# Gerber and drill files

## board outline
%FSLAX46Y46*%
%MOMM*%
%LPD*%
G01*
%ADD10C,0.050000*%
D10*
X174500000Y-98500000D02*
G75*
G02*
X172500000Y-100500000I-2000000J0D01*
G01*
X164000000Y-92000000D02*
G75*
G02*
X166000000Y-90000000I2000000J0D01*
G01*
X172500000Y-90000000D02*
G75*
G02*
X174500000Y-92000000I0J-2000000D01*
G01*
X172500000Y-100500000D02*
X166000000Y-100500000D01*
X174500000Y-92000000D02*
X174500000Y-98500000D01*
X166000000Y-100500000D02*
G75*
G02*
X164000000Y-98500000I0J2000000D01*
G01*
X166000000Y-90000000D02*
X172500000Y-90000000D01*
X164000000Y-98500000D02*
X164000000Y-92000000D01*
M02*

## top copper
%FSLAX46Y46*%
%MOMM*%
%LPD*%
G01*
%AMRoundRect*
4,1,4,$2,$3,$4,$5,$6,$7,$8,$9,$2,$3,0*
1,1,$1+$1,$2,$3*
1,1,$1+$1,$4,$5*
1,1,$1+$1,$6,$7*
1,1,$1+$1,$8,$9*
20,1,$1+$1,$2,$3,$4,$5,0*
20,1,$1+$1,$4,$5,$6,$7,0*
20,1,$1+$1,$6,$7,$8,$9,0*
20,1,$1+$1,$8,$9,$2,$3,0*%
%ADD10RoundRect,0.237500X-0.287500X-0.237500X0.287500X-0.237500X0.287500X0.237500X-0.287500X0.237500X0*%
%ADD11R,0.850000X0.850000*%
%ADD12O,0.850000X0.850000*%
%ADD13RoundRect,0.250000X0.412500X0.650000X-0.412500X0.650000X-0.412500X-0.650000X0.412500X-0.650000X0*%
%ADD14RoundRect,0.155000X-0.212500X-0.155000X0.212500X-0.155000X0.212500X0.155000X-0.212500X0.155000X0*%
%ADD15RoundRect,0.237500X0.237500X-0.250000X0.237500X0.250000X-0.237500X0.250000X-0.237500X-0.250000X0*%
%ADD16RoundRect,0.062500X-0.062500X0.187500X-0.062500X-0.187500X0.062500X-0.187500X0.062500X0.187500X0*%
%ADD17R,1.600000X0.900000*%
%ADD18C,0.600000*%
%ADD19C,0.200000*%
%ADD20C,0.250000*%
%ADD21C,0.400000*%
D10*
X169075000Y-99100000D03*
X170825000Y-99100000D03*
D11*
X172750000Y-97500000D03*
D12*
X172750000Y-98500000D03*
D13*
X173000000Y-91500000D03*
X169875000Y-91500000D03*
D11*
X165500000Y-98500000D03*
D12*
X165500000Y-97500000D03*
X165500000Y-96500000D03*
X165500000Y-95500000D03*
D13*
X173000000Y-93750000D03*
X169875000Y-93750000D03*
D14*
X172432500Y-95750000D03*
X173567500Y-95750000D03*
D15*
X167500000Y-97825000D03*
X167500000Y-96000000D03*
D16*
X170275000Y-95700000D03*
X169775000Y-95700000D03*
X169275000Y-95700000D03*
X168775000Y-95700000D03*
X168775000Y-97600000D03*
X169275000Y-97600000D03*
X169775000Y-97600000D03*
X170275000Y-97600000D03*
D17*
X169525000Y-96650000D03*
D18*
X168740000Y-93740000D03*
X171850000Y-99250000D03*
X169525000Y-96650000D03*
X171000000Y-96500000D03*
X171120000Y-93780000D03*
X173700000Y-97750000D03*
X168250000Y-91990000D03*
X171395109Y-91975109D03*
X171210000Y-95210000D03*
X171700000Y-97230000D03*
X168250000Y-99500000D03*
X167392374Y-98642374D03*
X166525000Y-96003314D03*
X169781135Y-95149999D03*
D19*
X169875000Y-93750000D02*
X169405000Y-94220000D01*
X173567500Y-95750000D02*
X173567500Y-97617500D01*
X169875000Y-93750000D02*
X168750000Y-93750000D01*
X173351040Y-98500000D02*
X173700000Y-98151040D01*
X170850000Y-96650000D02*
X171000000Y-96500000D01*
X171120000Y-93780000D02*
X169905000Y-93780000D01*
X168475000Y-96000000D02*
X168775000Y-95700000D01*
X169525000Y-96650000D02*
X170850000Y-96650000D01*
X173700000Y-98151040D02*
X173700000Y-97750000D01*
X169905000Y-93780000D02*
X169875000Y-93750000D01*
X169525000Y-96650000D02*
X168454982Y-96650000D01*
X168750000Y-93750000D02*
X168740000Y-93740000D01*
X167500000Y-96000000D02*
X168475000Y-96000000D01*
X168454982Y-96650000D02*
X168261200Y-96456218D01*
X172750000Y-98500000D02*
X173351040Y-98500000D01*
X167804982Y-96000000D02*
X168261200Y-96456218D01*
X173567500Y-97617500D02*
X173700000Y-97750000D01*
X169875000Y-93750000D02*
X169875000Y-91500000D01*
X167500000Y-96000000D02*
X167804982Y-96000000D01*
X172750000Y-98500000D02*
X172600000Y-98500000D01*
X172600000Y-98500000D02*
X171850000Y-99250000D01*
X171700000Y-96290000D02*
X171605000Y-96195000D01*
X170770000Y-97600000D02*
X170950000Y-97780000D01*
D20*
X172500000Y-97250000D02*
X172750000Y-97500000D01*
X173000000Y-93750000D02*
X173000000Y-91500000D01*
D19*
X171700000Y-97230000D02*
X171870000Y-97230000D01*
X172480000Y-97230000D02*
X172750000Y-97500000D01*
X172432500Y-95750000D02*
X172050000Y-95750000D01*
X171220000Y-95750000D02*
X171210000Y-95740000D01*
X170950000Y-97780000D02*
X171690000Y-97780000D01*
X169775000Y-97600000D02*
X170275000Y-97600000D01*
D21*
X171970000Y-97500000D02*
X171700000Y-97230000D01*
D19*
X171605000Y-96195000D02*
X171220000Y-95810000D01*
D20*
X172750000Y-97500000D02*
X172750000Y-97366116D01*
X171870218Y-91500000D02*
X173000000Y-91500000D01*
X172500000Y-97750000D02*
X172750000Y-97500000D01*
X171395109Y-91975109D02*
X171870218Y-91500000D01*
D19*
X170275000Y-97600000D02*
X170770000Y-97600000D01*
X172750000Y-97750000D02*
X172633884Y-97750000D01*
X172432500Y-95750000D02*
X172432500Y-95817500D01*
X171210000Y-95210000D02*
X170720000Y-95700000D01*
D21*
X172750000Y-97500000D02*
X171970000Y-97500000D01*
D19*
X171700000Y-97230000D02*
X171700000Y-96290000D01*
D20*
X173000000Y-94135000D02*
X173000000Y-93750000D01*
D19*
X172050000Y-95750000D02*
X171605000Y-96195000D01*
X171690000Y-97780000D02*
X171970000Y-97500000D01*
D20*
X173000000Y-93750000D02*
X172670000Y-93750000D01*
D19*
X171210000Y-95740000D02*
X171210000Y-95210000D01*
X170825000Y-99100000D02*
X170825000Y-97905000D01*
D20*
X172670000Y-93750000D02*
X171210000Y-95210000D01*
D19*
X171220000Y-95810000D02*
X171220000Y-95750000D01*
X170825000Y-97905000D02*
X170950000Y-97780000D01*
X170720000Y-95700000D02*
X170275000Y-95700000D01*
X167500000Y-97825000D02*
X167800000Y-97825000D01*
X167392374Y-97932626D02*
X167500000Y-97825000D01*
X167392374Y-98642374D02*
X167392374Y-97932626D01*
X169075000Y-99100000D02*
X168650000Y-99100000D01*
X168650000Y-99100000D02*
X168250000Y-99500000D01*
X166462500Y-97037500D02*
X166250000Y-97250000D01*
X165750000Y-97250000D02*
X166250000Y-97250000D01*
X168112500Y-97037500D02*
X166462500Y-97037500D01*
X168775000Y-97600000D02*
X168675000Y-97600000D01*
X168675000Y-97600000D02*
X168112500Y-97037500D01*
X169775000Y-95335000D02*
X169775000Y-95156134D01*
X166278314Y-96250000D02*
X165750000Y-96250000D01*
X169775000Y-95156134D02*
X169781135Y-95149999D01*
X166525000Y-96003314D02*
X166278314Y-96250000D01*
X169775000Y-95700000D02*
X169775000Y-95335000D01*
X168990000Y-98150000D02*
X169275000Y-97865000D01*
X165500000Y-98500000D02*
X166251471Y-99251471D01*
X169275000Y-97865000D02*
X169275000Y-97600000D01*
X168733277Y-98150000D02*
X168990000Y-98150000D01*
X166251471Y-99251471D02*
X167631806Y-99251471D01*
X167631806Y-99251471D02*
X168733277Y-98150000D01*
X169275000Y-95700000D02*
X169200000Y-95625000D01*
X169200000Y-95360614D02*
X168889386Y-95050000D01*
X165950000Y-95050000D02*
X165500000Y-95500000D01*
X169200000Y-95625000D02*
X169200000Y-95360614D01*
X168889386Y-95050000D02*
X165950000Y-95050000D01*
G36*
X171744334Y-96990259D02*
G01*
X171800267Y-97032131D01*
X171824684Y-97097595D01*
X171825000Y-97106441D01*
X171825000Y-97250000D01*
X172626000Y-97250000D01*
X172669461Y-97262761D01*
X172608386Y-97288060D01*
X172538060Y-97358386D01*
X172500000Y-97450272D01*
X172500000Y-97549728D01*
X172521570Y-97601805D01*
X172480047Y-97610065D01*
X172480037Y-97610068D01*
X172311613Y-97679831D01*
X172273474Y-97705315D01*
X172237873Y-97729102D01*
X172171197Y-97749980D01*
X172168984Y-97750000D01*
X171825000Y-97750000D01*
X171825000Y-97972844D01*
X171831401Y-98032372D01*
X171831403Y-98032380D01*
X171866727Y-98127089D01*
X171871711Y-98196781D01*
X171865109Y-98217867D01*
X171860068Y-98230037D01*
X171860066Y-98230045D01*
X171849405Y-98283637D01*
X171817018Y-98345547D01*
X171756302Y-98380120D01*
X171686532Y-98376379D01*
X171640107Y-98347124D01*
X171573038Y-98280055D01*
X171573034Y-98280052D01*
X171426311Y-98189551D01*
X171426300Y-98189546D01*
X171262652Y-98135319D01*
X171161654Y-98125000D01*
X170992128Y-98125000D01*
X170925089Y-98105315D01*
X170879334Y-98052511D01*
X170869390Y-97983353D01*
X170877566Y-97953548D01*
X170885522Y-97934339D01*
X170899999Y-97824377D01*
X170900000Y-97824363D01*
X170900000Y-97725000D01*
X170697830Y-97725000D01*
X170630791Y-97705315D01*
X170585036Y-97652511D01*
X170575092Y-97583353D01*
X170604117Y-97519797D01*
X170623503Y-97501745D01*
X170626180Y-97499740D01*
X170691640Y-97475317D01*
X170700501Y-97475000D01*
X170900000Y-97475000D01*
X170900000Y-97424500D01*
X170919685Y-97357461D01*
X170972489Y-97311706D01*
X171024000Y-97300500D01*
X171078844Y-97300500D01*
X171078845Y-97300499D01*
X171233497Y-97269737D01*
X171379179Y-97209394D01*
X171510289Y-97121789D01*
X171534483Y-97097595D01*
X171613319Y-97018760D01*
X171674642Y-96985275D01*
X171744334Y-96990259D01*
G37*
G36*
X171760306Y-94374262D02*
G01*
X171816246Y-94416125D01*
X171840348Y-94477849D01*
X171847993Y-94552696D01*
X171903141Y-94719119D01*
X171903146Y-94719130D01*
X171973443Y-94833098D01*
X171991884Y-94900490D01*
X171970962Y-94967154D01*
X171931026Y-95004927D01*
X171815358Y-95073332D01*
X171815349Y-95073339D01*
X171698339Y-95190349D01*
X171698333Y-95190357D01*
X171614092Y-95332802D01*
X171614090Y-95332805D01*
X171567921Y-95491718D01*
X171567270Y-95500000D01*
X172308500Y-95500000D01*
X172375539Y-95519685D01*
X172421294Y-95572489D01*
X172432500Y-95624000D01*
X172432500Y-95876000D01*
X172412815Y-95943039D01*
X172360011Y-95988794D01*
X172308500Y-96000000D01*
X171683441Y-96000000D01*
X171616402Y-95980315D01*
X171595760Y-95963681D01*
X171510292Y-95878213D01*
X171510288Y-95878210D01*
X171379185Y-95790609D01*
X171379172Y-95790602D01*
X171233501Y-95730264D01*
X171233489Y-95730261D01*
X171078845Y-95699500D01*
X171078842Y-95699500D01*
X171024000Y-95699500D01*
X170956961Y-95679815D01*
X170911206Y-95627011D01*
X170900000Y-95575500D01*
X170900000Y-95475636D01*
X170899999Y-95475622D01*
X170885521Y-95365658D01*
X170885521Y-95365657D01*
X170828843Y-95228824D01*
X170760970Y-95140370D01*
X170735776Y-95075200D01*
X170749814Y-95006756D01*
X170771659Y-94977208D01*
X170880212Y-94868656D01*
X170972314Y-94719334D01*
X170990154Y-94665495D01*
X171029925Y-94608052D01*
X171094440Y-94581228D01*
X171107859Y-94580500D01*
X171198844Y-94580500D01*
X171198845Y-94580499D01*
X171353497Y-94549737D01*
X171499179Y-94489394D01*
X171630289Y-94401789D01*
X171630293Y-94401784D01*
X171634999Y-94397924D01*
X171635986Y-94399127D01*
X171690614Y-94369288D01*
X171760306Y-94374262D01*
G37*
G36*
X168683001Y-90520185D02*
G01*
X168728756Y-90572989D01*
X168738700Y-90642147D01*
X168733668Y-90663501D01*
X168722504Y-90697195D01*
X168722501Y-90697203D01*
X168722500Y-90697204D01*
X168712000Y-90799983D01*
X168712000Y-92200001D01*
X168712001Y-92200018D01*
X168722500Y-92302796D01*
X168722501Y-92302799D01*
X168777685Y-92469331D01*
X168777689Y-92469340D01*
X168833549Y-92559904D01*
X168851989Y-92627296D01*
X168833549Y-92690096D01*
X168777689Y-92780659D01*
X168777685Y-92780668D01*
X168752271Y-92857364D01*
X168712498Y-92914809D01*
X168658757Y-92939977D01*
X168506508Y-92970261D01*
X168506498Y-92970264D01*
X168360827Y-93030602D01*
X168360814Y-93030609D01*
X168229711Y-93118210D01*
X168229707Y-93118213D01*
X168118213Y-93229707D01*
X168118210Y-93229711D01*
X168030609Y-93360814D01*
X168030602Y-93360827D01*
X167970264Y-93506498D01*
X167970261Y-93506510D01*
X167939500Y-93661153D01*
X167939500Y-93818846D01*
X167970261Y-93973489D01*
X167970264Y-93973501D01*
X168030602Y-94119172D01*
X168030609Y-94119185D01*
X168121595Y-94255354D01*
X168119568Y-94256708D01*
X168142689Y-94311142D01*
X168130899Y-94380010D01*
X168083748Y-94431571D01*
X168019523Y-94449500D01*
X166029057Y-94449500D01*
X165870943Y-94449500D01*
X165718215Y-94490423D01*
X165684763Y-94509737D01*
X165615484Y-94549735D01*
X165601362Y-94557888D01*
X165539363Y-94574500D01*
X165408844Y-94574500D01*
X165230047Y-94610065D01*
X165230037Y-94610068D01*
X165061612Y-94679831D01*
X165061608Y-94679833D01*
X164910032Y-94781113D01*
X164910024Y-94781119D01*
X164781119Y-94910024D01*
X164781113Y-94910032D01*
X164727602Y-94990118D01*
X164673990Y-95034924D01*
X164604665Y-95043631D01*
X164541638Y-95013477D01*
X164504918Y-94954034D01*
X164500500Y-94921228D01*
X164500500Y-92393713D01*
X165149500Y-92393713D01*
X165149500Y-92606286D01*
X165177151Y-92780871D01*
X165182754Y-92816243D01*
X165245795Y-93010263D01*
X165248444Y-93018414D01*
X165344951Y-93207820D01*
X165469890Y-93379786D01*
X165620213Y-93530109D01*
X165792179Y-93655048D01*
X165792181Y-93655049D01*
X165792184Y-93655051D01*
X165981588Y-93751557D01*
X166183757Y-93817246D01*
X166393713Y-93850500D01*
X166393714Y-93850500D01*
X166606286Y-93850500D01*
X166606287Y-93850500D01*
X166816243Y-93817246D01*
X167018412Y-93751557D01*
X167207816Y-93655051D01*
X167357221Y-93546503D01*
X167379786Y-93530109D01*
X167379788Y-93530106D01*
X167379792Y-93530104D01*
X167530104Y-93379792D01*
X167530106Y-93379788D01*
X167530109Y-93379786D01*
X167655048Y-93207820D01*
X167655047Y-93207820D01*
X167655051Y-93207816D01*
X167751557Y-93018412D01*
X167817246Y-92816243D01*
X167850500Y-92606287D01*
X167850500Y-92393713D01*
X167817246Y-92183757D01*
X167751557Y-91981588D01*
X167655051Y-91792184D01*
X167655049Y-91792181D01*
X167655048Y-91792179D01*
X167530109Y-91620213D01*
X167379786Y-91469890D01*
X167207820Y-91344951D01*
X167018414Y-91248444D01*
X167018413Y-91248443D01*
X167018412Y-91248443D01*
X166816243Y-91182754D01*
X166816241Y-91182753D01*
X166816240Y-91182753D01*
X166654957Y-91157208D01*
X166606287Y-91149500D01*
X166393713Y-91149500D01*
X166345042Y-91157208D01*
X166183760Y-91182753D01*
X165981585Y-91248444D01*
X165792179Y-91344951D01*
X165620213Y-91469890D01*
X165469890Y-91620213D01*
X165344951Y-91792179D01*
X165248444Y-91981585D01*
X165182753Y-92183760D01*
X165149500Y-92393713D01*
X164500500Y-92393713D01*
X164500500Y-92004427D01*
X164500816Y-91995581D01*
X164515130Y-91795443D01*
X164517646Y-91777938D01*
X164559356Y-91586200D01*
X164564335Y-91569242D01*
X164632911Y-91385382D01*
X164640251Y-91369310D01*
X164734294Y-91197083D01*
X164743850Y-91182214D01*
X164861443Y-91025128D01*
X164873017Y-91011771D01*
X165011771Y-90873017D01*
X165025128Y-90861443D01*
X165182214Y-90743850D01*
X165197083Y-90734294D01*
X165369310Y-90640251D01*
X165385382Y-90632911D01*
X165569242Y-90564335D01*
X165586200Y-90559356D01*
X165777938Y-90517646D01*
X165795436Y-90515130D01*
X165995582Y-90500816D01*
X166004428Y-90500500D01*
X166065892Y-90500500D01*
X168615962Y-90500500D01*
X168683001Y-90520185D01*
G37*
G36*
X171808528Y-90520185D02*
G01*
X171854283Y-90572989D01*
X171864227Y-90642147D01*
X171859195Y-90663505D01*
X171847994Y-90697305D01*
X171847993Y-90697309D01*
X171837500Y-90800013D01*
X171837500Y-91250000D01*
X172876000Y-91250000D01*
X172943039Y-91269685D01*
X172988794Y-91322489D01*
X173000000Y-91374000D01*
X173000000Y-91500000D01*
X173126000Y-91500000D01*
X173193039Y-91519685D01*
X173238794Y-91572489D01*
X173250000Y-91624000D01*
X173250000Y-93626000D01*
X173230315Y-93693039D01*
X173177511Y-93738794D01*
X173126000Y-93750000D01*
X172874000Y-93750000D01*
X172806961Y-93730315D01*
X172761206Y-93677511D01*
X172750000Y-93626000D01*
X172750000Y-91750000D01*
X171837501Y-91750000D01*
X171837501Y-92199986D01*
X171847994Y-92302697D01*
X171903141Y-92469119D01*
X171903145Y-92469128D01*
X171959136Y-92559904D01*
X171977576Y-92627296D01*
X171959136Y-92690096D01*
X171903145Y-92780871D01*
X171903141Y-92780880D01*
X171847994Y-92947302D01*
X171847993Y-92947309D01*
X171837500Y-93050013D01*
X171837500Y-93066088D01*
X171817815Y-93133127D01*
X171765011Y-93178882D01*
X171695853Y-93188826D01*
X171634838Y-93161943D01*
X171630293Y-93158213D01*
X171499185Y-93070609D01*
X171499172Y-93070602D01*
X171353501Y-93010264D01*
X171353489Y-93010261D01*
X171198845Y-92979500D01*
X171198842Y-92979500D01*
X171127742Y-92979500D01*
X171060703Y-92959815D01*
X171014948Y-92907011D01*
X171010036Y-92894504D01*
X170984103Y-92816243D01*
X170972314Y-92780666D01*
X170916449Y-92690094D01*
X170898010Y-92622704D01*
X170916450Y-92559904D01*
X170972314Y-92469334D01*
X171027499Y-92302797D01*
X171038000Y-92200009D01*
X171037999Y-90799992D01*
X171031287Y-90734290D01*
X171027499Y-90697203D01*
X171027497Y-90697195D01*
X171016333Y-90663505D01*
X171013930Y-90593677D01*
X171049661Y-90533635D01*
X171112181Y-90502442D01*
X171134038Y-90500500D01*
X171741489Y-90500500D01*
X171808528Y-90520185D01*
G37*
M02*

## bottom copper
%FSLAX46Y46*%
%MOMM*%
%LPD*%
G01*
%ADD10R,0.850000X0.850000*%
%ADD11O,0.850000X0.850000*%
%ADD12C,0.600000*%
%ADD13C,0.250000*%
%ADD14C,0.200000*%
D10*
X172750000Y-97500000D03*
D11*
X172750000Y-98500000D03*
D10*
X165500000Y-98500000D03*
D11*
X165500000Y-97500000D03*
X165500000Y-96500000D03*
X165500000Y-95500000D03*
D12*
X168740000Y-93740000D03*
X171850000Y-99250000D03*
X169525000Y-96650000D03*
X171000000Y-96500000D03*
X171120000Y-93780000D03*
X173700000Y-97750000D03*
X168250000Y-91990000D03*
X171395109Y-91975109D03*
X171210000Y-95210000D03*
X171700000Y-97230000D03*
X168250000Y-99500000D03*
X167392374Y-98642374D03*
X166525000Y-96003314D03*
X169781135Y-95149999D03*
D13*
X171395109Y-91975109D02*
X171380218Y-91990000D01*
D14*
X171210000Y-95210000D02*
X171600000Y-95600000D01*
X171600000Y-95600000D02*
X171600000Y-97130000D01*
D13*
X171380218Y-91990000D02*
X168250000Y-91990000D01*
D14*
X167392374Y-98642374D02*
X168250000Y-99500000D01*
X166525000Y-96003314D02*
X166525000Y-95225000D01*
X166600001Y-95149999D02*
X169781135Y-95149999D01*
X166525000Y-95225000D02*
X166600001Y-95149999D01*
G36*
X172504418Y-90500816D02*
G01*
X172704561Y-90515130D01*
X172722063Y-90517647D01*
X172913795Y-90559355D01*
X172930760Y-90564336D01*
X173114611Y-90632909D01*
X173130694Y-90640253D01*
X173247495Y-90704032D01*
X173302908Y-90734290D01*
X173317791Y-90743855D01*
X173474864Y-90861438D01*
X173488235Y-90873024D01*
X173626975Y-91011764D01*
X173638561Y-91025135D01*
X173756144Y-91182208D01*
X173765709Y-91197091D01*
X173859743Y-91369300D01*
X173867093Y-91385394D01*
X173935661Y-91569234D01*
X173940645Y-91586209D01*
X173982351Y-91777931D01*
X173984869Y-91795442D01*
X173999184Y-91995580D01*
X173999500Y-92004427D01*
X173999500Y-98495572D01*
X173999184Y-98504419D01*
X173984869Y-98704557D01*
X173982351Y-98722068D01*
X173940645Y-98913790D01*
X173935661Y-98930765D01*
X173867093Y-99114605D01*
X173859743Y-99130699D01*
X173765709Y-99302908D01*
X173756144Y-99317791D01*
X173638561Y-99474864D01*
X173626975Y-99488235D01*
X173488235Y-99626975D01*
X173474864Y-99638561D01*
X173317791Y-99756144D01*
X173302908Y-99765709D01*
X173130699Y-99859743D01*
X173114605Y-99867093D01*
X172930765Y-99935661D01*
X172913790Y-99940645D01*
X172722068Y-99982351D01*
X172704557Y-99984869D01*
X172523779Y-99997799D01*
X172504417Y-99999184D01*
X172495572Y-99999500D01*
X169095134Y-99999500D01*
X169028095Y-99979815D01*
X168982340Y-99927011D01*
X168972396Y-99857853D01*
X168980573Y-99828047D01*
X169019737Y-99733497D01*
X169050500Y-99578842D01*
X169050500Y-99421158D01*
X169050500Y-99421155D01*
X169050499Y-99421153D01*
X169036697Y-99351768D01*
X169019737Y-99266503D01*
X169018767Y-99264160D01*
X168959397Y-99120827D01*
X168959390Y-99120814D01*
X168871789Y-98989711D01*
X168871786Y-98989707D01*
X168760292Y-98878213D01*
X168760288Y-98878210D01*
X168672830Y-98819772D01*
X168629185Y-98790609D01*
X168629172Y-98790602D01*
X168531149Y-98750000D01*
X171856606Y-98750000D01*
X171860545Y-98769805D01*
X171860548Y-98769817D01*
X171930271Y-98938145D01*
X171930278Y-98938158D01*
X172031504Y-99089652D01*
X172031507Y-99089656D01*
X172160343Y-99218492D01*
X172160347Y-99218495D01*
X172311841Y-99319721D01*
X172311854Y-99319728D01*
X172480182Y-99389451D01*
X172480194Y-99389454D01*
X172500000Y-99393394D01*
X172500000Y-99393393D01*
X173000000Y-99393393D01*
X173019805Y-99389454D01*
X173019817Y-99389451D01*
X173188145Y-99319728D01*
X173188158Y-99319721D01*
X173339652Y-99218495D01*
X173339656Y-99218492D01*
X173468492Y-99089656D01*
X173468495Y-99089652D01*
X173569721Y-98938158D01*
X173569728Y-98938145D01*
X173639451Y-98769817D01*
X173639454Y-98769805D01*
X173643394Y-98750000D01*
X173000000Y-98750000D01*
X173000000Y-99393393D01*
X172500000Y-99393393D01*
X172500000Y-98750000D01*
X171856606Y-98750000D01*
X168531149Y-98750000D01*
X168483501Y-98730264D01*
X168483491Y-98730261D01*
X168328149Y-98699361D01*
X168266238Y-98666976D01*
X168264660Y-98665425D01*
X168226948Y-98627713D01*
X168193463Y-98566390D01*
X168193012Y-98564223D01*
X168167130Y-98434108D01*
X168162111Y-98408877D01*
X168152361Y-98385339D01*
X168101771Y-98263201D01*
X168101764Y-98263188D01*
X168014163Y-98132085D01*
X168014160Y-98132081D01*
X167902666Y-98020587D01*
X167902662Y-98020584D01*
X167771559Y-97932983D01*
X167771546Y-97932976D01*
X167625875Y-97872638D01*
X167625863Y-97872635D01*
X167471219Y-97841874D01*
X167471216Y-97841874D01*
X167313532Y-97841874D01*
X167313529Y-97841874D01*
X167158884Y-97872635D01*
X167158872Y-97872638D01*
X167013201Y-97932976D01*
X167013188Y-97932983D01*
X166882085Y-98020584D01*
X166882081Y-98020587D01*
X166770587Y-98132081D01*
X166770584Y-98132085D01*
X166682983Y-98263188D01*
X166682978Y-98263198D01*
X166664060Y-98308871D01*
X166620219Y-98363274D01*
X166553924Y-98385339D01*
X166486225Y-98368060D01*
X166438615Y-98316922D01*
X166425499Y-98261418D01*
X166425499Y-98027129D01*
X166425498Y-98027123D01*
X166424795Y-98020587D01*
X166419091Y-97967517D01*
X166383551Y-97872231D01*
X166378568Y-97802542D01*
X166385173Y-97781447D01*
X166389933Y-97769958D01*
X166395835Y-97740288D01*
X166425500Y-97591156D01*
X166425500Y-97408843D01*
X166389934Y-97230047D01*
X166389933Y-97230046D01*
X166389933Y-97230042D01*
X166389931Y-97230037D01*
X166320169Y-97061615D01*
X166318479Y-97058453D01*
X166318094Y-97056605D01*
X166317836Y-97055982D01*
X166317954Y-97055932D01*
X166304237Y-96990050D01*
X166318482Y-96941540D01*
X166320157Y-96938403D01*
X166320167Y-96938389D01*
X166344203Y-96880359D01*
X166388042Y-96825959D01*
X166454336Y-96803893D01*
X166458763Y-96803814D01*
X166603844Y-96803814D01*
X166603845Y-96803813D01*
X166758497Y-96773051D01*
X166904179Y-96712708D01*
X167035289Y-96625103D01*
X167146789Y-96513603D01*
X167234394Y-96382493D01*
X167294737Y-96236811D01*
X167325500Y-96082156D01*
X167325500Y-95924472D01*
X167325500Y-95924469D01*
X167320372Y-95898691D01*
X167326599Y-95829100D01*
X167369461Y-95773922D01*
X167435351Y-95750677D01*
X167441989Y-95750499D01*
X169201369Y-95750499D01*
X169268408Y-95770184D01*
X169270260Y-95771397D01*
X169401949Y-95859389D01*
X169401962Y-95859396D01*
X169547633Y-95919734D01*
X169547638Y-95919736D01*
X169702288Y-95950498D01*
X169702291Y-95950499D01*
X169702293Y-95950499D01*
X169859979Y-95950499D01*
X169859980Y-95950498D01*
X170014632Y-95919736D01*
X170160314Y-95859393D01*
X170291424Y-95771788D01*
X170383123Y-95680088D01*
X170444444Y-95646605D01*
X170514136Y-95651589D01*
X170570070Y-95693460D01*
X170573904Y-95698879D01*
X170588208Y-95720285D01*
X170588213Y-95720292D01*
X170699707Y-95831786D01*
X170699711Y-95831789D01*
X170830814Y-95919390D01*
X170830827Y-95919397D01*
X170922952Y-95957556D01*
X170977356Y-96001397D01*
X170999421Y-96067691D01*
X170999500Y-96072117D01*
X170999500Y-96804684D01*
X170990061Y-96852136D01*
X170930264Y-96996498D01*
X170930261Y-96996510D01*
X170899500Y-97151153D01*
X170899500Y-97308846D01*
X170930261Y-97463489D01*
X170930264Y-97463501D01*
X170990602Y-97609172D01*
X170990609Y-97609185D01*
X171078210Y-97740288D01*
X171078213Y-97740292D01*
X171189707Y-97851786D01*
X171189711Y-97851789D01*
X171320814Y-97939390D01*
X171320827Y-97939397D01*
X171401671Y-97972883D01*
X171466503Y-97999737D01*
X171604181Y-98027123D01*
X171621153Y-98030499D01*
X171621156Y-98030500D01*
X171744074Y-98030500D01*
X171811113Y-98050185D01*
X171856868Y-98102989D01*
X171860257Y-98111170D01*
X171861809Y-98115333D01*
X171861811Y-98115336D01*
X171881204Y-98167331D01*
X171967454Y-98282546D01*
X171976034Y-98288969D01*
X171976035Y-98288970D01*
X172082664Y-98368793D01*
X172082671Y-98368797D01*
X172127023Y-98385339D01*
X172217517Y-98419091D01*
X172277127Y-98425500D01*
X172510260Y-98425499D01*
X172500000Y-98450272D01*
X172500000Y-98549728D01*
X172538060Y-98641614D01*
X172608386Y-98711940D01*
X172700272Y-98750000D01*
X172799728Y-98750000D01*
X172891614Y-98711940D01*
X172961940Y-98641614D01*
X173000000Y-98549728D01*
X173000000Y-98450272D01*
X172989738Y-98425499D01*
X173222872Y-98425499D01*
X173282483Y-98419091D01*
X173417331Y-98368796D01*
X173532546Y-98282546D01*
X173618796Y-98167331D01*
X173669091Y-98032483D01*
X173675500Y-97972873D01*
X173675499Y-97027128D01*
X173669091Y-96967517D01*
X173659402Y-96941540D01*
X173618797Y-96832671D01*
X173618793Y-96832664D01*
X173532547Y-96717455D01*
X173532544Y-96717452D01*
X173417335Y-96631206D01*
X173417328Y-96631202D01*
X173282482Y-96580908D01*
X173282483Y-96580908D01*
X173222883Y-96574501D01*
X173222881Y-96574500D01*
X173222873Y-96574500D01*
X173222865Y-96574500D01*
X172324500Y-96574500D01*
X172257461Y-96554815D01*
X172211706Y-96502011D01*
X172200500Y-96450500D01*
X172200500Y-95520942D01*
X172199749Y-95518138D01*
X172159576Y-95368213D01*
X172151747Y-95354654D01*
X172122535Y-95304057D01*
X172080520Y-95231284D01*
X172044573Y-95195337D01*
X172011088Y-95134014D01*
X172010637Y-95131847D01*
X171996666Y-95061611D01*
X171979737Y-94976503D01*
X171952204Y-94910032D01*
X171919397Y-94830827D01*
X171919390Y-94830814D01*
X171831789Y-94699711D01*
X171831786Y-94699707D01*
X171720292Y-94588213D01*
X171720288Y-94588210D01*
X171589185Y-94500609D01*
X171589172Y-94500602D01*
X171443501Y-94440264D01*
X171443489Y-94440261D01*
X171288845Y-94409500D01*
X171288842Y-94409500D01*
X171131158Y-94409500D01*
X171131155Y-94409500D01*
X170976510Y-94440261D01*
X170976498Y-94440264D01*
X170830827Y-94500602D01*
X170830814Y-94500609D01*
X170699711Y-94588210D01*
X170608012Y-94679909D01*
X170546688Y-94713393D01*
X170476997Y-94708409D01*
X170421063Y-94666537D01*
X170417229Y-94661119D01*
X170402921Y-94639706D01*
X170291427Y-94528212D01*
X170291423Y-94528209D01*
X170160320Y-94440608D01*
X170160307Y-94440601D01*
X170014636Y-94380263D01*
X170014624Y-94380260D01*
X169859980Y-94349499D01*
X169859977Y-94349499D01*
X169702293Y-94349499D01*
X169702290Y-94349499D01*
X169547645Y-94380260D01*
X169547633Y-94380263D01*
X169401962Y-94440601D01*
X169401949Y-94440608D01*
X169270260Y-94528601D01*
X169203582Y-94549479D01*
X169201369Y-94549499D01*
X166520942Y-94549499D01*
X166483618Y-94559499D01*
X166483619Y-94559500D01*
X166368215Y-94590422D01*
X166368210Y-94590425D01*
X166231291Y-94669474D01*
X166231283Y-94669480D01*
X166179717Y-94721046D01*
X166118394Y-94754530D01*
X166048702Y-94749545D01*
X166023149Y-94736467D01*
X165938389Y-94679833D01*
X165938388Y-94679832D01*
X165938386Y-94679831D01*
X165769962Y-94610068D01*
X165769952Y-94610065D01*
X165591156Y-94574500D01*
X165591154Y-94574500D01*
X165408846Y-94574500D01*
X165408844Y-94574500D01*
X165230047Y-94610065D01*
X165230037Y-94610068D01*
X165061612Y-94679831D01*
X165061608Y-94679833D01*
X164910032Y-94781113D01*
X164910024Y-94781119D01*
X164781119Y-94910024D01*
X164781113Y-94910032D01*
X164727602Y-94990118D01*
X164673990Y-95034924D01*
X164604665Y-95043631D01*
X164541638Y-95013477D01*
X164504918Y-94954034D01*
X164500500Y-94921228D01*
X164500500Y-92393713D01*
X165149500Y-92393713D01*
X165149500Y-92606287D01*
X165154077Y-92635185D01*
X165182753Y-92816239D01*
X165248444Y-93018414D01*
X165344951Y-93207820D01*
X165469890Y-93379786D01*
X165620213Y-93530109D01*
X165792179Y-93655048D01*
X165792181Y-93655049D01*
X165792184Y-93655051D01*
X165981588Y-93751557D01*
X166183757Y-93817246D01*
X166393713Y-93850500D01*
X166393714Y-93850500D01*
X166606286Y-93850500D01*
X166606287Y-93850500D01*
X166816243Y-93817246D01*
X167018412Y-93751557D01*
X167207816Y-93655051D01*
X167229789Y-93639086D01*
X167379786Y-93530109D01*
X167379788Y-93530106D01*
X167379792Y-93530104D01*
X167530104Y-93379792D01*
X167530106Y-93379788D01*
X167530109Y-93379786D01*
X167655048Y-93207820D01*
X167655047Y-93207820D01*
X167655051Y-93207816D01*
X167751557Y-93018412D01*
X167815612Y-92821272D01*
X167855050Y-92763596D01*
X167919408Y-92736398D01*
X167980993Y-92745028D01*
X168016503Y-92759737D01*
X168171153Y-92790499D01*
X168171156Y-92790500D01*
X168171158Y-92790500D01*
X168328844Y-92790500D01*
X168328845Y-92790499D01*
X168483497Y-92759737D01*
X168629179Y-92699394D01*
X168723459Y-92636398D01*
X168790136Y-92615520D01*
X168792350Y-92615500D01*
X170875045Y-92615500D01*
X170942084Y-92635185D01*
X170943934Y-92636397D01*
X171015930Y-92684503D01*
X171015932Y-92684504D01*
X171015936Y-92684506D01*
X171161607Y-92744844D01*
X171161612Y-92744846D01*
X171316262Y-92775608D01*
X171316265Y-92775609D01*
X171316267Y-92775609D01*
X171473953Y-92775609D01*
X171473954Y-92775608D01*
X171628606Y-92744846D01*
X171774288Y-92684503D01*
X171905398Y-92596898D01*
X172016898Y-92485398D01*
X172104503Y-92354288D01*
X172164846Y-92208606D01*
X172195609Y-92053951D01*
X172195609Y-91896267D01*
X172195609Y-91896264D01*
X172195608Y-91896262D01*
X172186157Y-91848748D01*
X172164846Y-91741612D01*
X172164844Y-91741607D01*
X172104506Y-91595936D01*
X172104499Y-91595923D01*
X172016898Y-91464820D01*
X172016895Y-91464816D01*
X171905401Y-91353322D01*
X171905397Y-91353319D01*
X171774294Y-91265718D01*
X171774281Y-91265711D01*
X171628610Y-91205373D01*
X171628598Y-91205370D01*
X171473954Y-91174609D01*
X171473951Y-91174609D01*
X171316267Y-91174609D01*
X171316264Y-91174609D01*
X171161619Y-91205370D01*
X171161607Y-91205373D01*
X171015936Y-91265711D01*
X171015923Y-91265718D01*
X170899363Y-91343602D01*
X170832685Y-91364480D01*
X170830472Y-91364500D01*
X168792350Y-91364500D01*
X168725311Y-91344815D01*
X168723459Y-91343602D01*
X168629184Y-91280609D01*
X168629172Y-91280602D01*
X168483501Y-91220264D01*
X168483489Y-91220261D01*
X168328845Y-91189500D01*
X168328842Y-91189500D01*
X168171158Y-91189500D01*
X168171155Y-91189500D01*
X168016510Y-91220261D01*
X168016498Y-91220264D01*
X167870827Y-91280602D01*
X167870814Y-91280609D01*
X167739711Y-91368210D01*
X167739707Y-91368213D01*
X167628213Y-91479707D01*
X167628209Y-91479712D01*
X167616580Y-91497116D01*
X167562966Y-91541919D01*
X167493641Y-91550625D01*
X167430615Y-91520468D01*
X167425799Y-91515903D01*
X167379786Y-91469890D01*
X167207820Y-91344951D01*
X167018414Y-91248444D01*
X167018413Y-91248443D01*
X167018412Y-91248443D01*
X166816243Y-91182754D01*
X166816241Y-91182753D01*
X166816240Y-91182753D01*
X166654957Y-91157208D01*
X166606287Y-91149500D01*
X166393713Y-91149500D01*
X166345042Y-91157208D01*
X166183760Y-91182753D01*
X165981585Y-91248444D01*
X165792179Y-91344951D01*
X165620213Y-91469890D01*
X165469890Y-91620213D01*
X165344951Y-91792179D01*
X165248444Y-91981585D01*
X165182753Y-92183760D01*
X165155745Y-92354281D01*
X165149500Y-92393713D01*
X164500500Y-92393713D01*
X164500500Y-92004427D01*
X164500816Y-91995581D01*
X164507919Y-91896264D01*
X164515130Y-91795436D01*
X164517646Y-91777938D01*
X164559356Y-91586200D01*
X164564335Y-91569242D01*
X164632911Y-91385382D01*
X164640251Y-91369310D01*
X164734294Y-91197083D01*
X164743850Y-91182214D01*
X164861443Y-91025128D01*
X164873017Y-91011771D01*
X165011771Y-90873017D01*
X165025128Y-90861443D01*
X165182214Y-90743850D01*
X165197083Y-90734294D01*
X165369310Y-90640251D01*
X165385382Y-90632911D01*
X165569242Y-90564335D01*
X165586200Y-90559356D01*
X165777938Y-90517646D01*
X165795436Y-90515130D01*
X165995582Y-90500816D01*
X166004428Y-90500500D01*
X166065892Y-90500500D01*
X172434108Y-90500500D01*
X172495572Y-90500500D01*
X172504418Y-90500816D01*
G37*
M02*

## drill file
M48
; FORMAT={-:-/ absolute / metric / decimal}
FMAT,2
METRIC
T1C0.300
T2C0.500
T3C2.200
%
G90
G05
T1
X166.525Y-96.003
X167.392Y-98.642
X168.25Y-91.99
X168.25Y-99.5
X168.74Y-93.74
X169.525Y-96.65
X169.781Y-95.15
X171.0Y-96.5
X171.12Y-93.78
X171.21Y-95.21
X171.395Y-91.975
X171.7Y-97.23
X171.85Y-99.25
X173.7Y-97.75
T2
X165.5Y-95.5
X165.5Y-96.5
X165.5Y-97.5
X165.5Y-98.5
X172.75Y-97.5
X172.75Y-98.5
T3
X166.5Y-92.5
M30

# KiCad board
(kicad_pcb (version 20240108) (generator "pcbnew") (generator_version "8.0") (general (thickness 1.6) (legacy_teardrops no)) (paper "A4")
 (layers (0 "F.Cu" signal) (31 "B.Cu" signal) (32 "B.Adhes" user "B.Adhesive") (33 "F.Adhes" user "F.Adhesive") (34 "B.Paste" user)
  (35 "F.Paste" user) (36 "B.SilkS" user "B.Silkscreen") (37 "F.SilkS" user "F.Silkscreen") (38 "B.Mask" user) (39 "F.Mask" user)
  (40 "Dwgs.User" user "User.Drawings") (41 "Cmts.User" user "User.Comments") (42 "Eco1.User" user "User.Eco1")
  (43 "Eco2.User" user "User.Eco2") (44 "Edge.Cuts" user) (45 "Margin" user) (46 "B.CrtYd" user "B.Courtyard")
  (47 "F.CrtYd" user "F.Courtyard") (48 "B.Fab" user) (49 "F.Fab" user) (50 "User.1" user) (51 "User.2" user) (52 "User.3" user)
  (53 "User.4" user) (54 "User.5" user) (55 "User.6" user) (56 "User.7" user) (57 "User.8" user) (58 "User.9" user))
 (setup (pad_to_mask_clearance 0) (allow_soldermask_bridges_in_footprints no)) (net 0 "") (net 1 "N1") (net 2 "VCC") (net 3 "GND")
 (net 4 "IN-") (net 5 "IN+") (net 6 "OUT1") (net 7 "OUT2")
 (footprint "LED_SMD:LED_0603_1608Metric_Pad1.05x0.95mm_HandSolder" (layer "F.Cu") (at 169.95 99.1)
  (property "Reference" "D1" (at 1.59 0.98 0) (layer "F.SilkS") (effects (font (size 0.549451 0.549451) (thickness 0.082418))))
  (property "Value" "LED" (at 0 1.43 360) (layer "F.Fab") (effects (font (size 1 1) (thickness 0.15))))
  (pad "1" smd roundrect (at -0.875 0) (size 1.05 0.95) (layers "F.Cu" "F.Paste" "F.Mask") (roundrect_rratio 0.25) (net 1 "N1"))
  (pad "2" smd roundrect (at 0.875 0) (size 1.05 0.95) (layers "F.Cu" "F.Paste" "F.Mask") (roundrect_rratio 0.25) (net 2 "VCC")))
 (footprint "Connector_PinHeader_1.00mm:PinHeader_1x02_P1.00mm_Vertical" (layer "F.Cu") (at 172.75 97.5)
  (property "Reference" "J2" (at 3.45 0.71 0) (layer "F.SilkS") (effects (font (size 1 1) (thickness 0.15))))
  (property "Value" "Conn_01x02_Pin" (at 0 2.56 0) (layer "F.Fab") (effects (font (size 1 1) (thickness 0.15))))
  (pad "1" thru_hole rect (at 0 0) (size 0.85 0.85) (drill 0.5) (layers "*.Cu" "*.Mask") (remove_unused_layers no) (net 2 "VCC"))
  (pad "2" thru_hole oval (at 0 1) (size 0.85 0.85) (drill 0.5) (layers "*.Cu" "*.Mask") (remove_unused_layers no) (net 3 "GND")))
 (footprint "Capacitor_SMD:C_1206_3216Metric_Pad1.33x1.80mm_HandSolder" (layer "F.Cu") (at 171.4375 91.5 180)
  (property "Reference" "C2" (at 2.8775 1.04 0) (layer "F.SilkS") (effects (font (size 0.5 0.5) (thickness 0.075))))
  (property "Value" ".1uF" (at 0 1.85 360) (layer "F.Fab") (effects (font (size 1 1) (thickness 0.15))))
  (pad "1" smd roundrect (at -1.5625 0 180) (size 1.325 1.8) (layers "F.Cu" "F.Paste" "F.Mask") (roundrect_rratio 0.188679) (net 2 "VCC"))
  (pad "2" smd roundrect (at 1.5625 0 180) (size 1.325 1.8) (layers "F.Cu" "F.Paste" "F.Mask") (roundrect_rratio 0.188679) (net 3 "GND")))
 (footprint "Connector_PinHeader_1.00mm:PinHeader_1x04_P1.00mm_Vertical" (layer "F.Cu") (at 165.5 98.5 180)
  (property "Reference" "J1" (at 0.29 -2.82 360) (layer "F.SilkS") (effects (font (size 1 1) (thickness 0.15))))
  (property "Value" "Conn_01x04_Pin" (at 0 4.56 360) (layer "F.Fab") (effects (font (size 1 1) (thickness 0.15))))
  (pad "1" thru_hole rect (at 0 0 180) (size 0.85 0.85) (drill 0.5) (layers "*.Cu" "*.Mask") (remove_unused_layers no) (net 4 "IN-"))
  (pad "2" thru_hole oval (at 0 1 180) (size 0.85 0.85) (drill 0.5) (layers "*.Cu" "*.Mask") (remove_unused_layers no) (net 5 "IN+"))
  (pad "3" thru_hole oval (at 0 2 180) (size 0.85 0.85) (drill 0.5) (layers "*.Cu" "*.Mask") (remove_unused_layers no) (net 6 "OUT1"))
  (pad "4" thru_hole oval (at 0 3 180) (size 0.85 0.85) (drill 0.5) (layers "*.Cu" "*.Mask") (remove_unused_layers no) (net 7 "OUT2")))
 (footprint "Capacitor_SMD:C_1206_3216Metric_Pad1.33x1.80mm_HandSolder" (layer "F.Cu") (at 171.4375 93.75 180)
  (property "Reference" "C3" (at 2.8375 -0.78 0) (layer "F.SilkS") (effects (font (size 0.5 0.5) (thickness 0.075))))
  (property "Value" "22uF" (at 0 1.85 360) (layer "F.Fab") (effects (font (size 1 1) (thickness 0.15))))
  (pad "1" smd roundrect (at -1.5625 0 180) (size 1.325 1.8) (layers "F.Cu" "F.Paste" "F.Mask") (roundrect_rratio 0.188679) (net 2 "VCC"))
  (pad "2" smd roundrect (at 1.5625 0 180) (size 1.325 1.8) (layers "F.Cu" "F.Paste" "F.Mask") (roundrect_rratio 0.188679) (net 3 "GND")))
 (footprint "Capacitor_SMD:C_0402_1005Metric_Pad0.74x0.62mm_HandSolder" (layer "F.Cu") (at 173 95.75)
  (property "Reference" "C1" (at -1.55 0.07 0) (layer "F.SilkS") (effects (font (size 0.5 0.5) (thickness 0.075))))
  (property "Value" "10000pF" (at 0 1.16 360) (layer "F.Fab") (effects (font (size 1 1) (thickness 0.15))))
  (pad "1" smd roundrect (at -0.5675 0) (size 0.735 0.62) (layers "F.Cu" "F.Paste" "F.Mask") (roundrect_rratio 0.25) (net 2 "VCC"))
  (pad "2" smd roundrect (at 0.5675 0) (size 0.735 0.62) (layers "F.Cu" "F.Paste" "F.Mask") (roundrect_rratio 0.25) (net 3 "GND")))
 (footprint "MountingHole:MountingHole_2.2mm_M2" (layer "F.Cu") (at 166.5 92.5)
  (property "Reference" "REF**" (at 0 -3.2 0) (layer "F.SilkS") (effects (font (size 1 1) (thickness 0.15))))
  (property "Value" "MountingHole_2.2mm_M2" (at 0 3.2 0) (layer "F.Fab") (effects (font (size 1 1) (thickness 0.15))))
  (pad "" np_thru_hole circle (at 0 0) (size 2.2 2.2) (drill 2.2) (layers "*.Cu" "*.Mask")))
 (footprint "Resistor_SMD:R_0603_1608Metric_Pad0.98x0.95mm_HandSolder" (layer "F.Cu") (at 167.5 96.9125 90)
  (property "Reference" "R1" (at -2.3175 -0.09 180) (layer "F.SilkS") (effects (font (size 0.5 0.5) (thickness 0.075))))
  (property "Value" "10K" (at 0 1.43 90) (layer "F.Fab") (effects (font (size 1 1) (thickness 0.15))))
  (pad "1" smd roundrect (at -0.9125 0 90) (size 0.975 0.95) (layers "F.Cu" "F.Paste" "F.Mask") (roundrect_rratio 0.25) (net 1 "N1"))
  (pad "2" smd roundrect (at 0.9125 0 90) (size 0.975 0.95) (layers "F.Cu" "F.Paste" "F.Mask") (roundrect_rratio 0.25) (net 3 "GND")))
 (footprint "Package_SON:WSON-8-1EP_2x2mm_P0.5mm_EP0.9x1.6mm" (layer "F.Cu") (at 169.525 96.65 -90)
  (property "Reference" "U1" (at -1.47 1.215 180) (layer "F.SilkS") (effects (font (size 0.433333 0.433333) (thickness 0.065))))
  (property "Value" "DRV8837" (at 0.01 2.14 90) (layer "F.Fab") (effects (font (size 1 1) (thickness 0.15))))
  (pad "" smd rect (at 0 -0.4 270) (size 0.75 0.65) (layers "F.Paste"))
  (pad "" smd rect (at 0 0.4 270) (size 0.75 0.65) (layers "F.Paste"))
  (pad "1" smd roundrect (at -0.95 -0.75 270) (size 0.5 0.25) (layers "F.Cu" "F.Paste" "F.Mask") (roundrect_rratio 0.25) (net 2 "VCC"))
  (pad "2" smd roundrect (at -0.95 -0.25 270) (size 0.5 0.25) (layers "F.Cu" "F.Paste" "F.Mask") (roundrect_rratio 0.25) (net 6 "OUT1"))
  (pad "3" smd roundrect (at -0.95 0.25 270) (size 0.5 0.25) (layers "F.Cu" "F.Paste" "F.Mask") (roundrect_rratio 0.25) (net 7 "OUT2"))
  (pad "4" smd roundrect (at -0.95 0.75 270) (size 0.5 0.25) (layers "F.Cu" "F.Paste" "F.Mask") (roundrect_rratio 0.25) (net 3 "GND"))
  (pad "5" smd roundrect (at 0.95 0.75 270) (size 0.5 0.25) (layers "F.Cu" "F.Paste" "F.Mask") (roundrect_rratio 0.25) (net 5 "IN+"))
  (pad "6" smd roundrect (at 0.95 0.25 270) (size 0.5 0.25) (layers "F.Cu" "F.Paste" "F.Mask") (roundrect_rratio 0.25) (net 4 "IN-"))
  (pad "7" smd roundrect (at 0.95 -0.25 270) (size 0.5 0.25) (layers "F.Cu" "F.Paste" "F.Mask") (roundrect_rratio 0.25) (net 2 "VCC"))
  (pad "8" smd roundrect (at 0.95 -0.75 270) (size 0.5 0.25) (layers "F.Cu" "F.Paste" "F.Mask") (roundrect_rratio 0.25) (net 2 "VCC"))
  (pad "9" smd rect (at 0 0 270) (size 0.9 1.6) (layers "F.Cu" "F.Mask") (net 3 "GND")))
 (gr_arc (start 174.5 98.5) (mid 173.914214 99.914214) (end 172.5 100.5) (stroke (width 0.05) (type default)) (layer "Edge.Cuts"))
 (gr_arc (start 164 92) (mid 164.585786 90.585786) (end 166 90) (stroke (width 0.05) (type default)) (layer "Edge.Cuts"))
 (gr_arc (start 172.5 90) (mid 173.914214 90.585786) (end 174.5 92) (stroke (width 0.05) (type default)) (layer "Edge.Cuts"))
 (gr_line (start 172.5 100.5) (end 166 100.5) (stroke (width 0.05) (type default)) (layer "Edge.Cuts"))
 (gr_line (start 174.5 92) (end 174.5 98.5) (stroke (width 0.05) (type default)) (layer "Edge.Cuts"))
 (gr_arc (start 166 100.5) (mid 164.585786 99.914214) (end 164 98.5) (stroke (width 0.05) (type default)) (layer "Edge.Cuts"))
 (gr_line (start 166 90) (end 172.5 90) (stroke (width 0.05) (type default)) (layer "Edge.Cuts"))
 (gr_line (start 164 98.5) (end 164 92) (stroke (width 0.05) (type default)) (layer "Edge.Cuts"))
 (segment (start 169.875 93.75) (end 169.405 94.22) (width 0.2) (layer "F.Cu") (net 3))
 (segment (start 173.5675 95.75) (end 173.5675 97.6175) (width 0.2) (layer "F.Cu") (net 3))
 (segment (start 169.875 93.75) (end 168.75 93.75) (width 0.2) (layer "F.Cu") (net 3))
 (segment (start 173.35104 98.5) (end 173.7 98.15104) (width 0.2) (layer "F.Cu") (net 3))
 (segment (start 170.85 96.65) (end 171 96.5) (width 0.2) (layer "F.Cu") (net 3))
 (segment (start 171.12 93.78) (end 169.905 93.78) (width 0.2) (layer "F.Cu") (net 3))
 (segment (start 168.475 96) (end 168.775 95.7) (width 0.2) (layer "F.Cu") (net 3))
 (segment (start 169.525 96.65) (end 170.85 96.65) (width 0.2) (layer "F.Cu") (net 3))
 (segment (start 173.7 98.15104) (end 173.7 97.75) (width 0.2) (layer "F.Cu") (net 3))
 (segment (start 169.905 93.78) (end 169.875 93.75) (width 0.2) (layer "F.Cu") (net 3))
 (segment (start 169.525 96.65) (end 168.454982 96.65) (width 0.2) (layer "F.Cu") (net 3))
 (segment (start 168.75 93.75) (end 168.74 93.74) (width 0.2) (layer "F.Cu") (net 3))
 (segment (start 167.5 96) (end 168.475 96) (width 0.2) (layer "F.Cu") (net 3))
 (segment (start 168.454982 96.65) (end 168.2612 96.456218) (width 0.2) (layer "F.Cu") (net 3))
 (segment (start 172.75 98.5) (end 173.35104 98.5) (width 0.2) (layer "F.Cu") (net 3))
 (segment (start 167.804982 96) (end 168.2612 96.456218) (width 0.2) (layer "F.Cu") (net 3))
 (segment (start 173.5675 97.6175) (end 173.7 97.75) (width 0.2) (layer "F.Cu") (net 3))
 (segment (start 169.875 93.75) (end 169.875 91.5) (width 0.2) (layer "F.Cu") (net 3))
 (segment (start 167.5 96) (end 167.804982 96) (width 0.2) (layer "F.Cu") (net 3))
 (segment (start 172.75 98.5) (end 172.6 98.5) (width 0.2) (layer "F.Cu") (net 3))
 (segment (start 172.6 98.5) (end 171.85 99.25) (width 0.2) (layer "F.Cu") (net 3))
 (via (at 168.74 93.74) (size 0.6) (drill 0.3) (layers "F.Cu" "B.Cu") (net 3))
 (via (at 171.85 99.25) (size 0.6) (drill 0.3) (layers "F.Cu" "B.Cu") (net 3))
 (via (at 169.525 96.65) (size 0.6) (drill 0.3) (layers "F.Cu" "B.Cu") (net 3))
 (via (at 171 96.5) (size 0.6) (drill 0.3) (layers "F.Cu" "B.Cu") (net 3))
 (via (at 171.12 93.78) (size 0.6) (drill 0.3) (layers "F.Cu" "B.Cu") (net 3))
 (via (at 173.7 97.75) (size 0.6) (drill 0.3) (layers "F.Cu" "B.Cu") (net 3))
 (segment (start 171.7 96.29) (end 171.605 96.195) (width 0.2) (layer "F.Cu") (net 2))
 (segment (start 170.77 97.6) (end 170.95 97.78) (width 0.2) (layer "F.Cu") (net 2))
 (segment (start 172.5 97.25) (end 172.75 97.5) (width 0.25) (layer "F.Cu") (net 2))
 (segment (start 173 93.75) (end 173 91.5) (width 0.25) (layer "F.Cu") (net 2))
 (segment (start 171.7 97.23) (end 171.87 97.23) (width 0.2) (layer "F.Cu") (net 2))
 (segment (start 172.48 97.23) (end 172.75 97.5) (width 0.2) (layer "F.Cu") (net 2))
 (segment (start 172.4325 95.75) (end 172.05 95.75) (width 0.2) (layer "F.Cu") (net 2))
 (segment (start 171.22 95.75) (end 171.21 95.74) (width 0.2) (layer "F.Cu") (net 2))
 (segment (start 170.95 97.78) (end 171.69 97.78) (width 0.2) (layer "F.Cu") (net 2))
 (segment (start 169.775 97.6) (end 170.275 97.6) (width 0.2) (layer "F.Cu") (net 2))
 (segment (start 171.97 97.5) (end 171.7 97.23) (width 0.4) (layer "F.Cu") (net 2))
 (segment (start 171.605 96.195) (end 171.22 95.81) (width 0.2) (layer "F.Cu") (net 2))
 (segment (start 172.75 97.5) (end 172.75 97.366116) (width 0.25) (layer "F.Cu") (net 2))
 (segment (start 171.870218 91.5) (end 173 91.5) (width 0.25) (layer "F.Cu") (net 2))
 (segment (start 172.5 97.75) (end 172.75 97.5) (width 0.25) (layer "F.Cu") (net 2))
 (segment (start 171.395109 91.975109) (end 171.870218 91.5) (width 0.25) (layer "F.Cu") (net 2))
 (segment (start 170.275 97.6) (end 170.77 97.6) (width 0.2) (layer "F.Cu") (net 2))
 (segment (start 172.75 97.75) (end 172.633884 97.75) (width 0.2) (layer "F.Cu") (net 2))
 (segment (start 172.4325 95.75) (end 172.4325 95.8175) (width 0.2) (layer "F.Cu") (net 2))
 (segment (start 171.21 95.21) (end 170.72 95.7) (width 0.2) (layer "F.Cu") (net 2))
 (segment (start 172.75 97.5) (end 171.97 97.5) (width 0.4) (layer "F.Cu") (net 2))
 (segment (start 171.7 97.23) (end 171.7 96.29) (width 0.2) (layer "F.Cu") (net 2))
 (segment (start 173 94.135) (end 173 93.75) (width 0.25) (layer "F.Cu") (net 2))
 (segment (start 172.05 95.75) (end 171.605 96.195) (width 0.2) (layer "F.Cu") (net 2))
 (segment (start 171.69 97.78) (end 171.97 97.5) (width 0.2) (layer "F.Cu") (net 2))
 (segment (start 173 93.75) (end 172.67 93.75) (width 0.25) (layer "F.Cu") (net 2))
 (segment (start 171.21 95.74) (end 171.21 95.21) (width 0.2) (layer "F.Cu") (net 2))
 (segment (start 170.825 99.1) (end 170.825 97.905) (width 0.2) (layer "F.Cu") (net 2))
 (segment (start 172.67 93.75) (end 171.21 95.21) (width 0.25) (layer "F.Cu") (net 2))
 (segment (start 171.22 95.81) (end 171.22 95.75) (width 0.2) (layer "F.Cu") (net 2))
 (segment (start 170.825 97.905) (end 170.95 97.78) (width 0.2) (layer "F.Cu") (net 2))
 (segment (start 170.72 95.7) (end 170.275 95.7) (width 0.2) (layer "F.Cu") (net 2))
 (via (at 168.25 91.99) (size 0.6) (drill 0.3) (layers "F.Cu" "B.Cu") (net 2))
 (via (at 171.395109 91.975109) (size 0.6) (drill 0.3) (layers "F.Cu" "B.Cu") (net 2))
 (via (at 171.21 95.21) (size 0.6) (drill 0.3) (layers "F.Cu" "B.Cu") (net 2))
 (via (at 171.7 97.23) (size 0.6) (drill 0.3) (layers "F.Cu" "B.Cu") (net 2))
 (segment (start 171.395109 91.975109) (end 171.380218 91.99) (width 0.25) (layer "B.Cu") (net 2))
 (segment (start 171.21 95.21) (end 171.6 95.6) (width 0.2) (layer "B.Cu") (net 2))
 (segment (start 171.6 95.6) (end 171.6 97.13) (width 0.2) (layer "B.Cu") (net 2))
 (segment (start 171.380218 91.99) (end 168.25 91.99) (width 0.25) (layer "B.Cu") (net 2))
 (segment (start 167.5 97.825) (end 167.8 97.825) (width 0.2) (layer "F.Cu") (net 1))
 (segment (start 167.392374 97.932626) (end 167.5 97.825) (width 0.2) (layer "F.Cu") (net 1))
 (segment (start 167.392374 98.642374) (end 167.392374 97.932626) (width 0.2) (layer "F.Cu") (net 1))
 (segment (start 169.075 99.1) (end 168.65 99.1) (width 0.2) (layer "F.Cu") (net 1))
 (segment (start 168.65 99.1) (end 168.25 99.5) (width 0.2) (layer "F.Cu") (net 1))
 (via (at 168.25 99.5) (size 0.6) (drill 0.3) (layers "F.Cu" "B.Cu") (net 1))
 (via (at 167.392374 98.642374) (size 0.6) (drill 0.3) (layers "F.Cu" "B.Cu") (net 1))
 (segment (start 167.392374 98.642374) (end 168.25 99.5) (width 0.2) (layer "B.Cu") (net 1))
 (segment (start 166.4625 97.0375) (end 166.25 97.25) (width 0.2) (layer "F.Cu") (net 5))
 (segment (start 165.75 97.25) (end 166.25 97.25) (width 0.2) (layer "F.Cu") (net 5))
 (segment (start 168.1125 97.0375) (end 166.4625 97.0375) (width 0.2) (layer "F.Cu") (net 5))
 (segment (start 168.775 97.6) (end 168.675 97.6) (width 0.2) (layer "F.Cu") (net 5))
 (segment (start 168.675 97.6) (end 168.1125 97.0375) (width 0.2) (layer "F.Cu") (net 5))
 (segment (start 169.775 95.335) (end 169.775 95.156134) (width 0.2) (layer "F.Cu") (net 6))
 (segment (start 166.278314 96.25) (end 165.75 96.25) (width 0.2) (layer "F.Cu") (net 6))
 (segment (start 169.775 95.156134) (end 169.781135 95.149999) (width 0.2) (layer "F.Cu") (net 6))
 (segment (start 166.525 96.003314) (end 166.278314 96.25) (width 0.2) (layer "F.Cu") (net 6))
 (segment (start 169.775 95.7) (end 169.775 95.335) (width 0.2) (layer "F.Cu") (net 6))
 (via (at 166.525 96.003314) (size 0.6) (drill 0.3) (layers "F.Cu" "B.Cu") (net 6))
 (via (at 169.781135 95.149999) (size 0.6) (drill 0.3) (layers "F.Cu" "B.Cu") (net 6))
 (segment (start 166.525 96.003314) (end 166.525 95.225) (width 0.2) (layer "B.Cu") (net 6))
 (segment (start 166.600001 95.149999) (end 169.781135 95.149999) (width 0.2) (layer "B.Cu") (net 6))
 (segment (start 166.525 95.225) (end 166.600001 95.149999) (width 0.2) (layer "B.Cu") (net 6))
 (segment (start 168.99 98.15) (end 169.275 97.865) (width 0.2) (layer "F.Cu") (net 4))
 (segment (start 165.5 98.5) (end 166.251471 99.251471) (width 0.2) (layer "F.Cu") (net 4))
 (segment (start 169.275 97.865) (end 169.275 97.6) (width 0.2) (layer "F.Cu") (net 4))
 (segment (start 168.733277 98.15) (end 168.99 98.15) (width 0.2) (layer "F.Cu") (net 4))
 (segment (start 166.251471 99.251471) (end 167.631806 99.251471) (width 0.2) (layer "F.Cu") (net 4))
 (segment (start 167.631806 99.251471) (end 168.733277 98.15) (width 0.2) (layer "F.Cu") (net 4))
 (segment (start 169.275 95.7) (end 169.2 95.625) (width 0.2) (layer "F.Cu") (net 7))
 (segment (start 169.2 95.360614) (end 168.889386 95.05) (width 0.2) (layer "F.Cu") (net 7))
 (segment (start 165.95 95.05) (end 165.5 95.5) (width 0.2) (layer "F.Cu") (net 7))
 (segment (start 169.2 95.625) (end 169.2 95.360614) (width 0.2) (layer "F.Cu") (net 7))
 (segment (start 168.889386 95.05) (end 165.95 95.05) (width 0.2) (layer "F.Cu") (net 7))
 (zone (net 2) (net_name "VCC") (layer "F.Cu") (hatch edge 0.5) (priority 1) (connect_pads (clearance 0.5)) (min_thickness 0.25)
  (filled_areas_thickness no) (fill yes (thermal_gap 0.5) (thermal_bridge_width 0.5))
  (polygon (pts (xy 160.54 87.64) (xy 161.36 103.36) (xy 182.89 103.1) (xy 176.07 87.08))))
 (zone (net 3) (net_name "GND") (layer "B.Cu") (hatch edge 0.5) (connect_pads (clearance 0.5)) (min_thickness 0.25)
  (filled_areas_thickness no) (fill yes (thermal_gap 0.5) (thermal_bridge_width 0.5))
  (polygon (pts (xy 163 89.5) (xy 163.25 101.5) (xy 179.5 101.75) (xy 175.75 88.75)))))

